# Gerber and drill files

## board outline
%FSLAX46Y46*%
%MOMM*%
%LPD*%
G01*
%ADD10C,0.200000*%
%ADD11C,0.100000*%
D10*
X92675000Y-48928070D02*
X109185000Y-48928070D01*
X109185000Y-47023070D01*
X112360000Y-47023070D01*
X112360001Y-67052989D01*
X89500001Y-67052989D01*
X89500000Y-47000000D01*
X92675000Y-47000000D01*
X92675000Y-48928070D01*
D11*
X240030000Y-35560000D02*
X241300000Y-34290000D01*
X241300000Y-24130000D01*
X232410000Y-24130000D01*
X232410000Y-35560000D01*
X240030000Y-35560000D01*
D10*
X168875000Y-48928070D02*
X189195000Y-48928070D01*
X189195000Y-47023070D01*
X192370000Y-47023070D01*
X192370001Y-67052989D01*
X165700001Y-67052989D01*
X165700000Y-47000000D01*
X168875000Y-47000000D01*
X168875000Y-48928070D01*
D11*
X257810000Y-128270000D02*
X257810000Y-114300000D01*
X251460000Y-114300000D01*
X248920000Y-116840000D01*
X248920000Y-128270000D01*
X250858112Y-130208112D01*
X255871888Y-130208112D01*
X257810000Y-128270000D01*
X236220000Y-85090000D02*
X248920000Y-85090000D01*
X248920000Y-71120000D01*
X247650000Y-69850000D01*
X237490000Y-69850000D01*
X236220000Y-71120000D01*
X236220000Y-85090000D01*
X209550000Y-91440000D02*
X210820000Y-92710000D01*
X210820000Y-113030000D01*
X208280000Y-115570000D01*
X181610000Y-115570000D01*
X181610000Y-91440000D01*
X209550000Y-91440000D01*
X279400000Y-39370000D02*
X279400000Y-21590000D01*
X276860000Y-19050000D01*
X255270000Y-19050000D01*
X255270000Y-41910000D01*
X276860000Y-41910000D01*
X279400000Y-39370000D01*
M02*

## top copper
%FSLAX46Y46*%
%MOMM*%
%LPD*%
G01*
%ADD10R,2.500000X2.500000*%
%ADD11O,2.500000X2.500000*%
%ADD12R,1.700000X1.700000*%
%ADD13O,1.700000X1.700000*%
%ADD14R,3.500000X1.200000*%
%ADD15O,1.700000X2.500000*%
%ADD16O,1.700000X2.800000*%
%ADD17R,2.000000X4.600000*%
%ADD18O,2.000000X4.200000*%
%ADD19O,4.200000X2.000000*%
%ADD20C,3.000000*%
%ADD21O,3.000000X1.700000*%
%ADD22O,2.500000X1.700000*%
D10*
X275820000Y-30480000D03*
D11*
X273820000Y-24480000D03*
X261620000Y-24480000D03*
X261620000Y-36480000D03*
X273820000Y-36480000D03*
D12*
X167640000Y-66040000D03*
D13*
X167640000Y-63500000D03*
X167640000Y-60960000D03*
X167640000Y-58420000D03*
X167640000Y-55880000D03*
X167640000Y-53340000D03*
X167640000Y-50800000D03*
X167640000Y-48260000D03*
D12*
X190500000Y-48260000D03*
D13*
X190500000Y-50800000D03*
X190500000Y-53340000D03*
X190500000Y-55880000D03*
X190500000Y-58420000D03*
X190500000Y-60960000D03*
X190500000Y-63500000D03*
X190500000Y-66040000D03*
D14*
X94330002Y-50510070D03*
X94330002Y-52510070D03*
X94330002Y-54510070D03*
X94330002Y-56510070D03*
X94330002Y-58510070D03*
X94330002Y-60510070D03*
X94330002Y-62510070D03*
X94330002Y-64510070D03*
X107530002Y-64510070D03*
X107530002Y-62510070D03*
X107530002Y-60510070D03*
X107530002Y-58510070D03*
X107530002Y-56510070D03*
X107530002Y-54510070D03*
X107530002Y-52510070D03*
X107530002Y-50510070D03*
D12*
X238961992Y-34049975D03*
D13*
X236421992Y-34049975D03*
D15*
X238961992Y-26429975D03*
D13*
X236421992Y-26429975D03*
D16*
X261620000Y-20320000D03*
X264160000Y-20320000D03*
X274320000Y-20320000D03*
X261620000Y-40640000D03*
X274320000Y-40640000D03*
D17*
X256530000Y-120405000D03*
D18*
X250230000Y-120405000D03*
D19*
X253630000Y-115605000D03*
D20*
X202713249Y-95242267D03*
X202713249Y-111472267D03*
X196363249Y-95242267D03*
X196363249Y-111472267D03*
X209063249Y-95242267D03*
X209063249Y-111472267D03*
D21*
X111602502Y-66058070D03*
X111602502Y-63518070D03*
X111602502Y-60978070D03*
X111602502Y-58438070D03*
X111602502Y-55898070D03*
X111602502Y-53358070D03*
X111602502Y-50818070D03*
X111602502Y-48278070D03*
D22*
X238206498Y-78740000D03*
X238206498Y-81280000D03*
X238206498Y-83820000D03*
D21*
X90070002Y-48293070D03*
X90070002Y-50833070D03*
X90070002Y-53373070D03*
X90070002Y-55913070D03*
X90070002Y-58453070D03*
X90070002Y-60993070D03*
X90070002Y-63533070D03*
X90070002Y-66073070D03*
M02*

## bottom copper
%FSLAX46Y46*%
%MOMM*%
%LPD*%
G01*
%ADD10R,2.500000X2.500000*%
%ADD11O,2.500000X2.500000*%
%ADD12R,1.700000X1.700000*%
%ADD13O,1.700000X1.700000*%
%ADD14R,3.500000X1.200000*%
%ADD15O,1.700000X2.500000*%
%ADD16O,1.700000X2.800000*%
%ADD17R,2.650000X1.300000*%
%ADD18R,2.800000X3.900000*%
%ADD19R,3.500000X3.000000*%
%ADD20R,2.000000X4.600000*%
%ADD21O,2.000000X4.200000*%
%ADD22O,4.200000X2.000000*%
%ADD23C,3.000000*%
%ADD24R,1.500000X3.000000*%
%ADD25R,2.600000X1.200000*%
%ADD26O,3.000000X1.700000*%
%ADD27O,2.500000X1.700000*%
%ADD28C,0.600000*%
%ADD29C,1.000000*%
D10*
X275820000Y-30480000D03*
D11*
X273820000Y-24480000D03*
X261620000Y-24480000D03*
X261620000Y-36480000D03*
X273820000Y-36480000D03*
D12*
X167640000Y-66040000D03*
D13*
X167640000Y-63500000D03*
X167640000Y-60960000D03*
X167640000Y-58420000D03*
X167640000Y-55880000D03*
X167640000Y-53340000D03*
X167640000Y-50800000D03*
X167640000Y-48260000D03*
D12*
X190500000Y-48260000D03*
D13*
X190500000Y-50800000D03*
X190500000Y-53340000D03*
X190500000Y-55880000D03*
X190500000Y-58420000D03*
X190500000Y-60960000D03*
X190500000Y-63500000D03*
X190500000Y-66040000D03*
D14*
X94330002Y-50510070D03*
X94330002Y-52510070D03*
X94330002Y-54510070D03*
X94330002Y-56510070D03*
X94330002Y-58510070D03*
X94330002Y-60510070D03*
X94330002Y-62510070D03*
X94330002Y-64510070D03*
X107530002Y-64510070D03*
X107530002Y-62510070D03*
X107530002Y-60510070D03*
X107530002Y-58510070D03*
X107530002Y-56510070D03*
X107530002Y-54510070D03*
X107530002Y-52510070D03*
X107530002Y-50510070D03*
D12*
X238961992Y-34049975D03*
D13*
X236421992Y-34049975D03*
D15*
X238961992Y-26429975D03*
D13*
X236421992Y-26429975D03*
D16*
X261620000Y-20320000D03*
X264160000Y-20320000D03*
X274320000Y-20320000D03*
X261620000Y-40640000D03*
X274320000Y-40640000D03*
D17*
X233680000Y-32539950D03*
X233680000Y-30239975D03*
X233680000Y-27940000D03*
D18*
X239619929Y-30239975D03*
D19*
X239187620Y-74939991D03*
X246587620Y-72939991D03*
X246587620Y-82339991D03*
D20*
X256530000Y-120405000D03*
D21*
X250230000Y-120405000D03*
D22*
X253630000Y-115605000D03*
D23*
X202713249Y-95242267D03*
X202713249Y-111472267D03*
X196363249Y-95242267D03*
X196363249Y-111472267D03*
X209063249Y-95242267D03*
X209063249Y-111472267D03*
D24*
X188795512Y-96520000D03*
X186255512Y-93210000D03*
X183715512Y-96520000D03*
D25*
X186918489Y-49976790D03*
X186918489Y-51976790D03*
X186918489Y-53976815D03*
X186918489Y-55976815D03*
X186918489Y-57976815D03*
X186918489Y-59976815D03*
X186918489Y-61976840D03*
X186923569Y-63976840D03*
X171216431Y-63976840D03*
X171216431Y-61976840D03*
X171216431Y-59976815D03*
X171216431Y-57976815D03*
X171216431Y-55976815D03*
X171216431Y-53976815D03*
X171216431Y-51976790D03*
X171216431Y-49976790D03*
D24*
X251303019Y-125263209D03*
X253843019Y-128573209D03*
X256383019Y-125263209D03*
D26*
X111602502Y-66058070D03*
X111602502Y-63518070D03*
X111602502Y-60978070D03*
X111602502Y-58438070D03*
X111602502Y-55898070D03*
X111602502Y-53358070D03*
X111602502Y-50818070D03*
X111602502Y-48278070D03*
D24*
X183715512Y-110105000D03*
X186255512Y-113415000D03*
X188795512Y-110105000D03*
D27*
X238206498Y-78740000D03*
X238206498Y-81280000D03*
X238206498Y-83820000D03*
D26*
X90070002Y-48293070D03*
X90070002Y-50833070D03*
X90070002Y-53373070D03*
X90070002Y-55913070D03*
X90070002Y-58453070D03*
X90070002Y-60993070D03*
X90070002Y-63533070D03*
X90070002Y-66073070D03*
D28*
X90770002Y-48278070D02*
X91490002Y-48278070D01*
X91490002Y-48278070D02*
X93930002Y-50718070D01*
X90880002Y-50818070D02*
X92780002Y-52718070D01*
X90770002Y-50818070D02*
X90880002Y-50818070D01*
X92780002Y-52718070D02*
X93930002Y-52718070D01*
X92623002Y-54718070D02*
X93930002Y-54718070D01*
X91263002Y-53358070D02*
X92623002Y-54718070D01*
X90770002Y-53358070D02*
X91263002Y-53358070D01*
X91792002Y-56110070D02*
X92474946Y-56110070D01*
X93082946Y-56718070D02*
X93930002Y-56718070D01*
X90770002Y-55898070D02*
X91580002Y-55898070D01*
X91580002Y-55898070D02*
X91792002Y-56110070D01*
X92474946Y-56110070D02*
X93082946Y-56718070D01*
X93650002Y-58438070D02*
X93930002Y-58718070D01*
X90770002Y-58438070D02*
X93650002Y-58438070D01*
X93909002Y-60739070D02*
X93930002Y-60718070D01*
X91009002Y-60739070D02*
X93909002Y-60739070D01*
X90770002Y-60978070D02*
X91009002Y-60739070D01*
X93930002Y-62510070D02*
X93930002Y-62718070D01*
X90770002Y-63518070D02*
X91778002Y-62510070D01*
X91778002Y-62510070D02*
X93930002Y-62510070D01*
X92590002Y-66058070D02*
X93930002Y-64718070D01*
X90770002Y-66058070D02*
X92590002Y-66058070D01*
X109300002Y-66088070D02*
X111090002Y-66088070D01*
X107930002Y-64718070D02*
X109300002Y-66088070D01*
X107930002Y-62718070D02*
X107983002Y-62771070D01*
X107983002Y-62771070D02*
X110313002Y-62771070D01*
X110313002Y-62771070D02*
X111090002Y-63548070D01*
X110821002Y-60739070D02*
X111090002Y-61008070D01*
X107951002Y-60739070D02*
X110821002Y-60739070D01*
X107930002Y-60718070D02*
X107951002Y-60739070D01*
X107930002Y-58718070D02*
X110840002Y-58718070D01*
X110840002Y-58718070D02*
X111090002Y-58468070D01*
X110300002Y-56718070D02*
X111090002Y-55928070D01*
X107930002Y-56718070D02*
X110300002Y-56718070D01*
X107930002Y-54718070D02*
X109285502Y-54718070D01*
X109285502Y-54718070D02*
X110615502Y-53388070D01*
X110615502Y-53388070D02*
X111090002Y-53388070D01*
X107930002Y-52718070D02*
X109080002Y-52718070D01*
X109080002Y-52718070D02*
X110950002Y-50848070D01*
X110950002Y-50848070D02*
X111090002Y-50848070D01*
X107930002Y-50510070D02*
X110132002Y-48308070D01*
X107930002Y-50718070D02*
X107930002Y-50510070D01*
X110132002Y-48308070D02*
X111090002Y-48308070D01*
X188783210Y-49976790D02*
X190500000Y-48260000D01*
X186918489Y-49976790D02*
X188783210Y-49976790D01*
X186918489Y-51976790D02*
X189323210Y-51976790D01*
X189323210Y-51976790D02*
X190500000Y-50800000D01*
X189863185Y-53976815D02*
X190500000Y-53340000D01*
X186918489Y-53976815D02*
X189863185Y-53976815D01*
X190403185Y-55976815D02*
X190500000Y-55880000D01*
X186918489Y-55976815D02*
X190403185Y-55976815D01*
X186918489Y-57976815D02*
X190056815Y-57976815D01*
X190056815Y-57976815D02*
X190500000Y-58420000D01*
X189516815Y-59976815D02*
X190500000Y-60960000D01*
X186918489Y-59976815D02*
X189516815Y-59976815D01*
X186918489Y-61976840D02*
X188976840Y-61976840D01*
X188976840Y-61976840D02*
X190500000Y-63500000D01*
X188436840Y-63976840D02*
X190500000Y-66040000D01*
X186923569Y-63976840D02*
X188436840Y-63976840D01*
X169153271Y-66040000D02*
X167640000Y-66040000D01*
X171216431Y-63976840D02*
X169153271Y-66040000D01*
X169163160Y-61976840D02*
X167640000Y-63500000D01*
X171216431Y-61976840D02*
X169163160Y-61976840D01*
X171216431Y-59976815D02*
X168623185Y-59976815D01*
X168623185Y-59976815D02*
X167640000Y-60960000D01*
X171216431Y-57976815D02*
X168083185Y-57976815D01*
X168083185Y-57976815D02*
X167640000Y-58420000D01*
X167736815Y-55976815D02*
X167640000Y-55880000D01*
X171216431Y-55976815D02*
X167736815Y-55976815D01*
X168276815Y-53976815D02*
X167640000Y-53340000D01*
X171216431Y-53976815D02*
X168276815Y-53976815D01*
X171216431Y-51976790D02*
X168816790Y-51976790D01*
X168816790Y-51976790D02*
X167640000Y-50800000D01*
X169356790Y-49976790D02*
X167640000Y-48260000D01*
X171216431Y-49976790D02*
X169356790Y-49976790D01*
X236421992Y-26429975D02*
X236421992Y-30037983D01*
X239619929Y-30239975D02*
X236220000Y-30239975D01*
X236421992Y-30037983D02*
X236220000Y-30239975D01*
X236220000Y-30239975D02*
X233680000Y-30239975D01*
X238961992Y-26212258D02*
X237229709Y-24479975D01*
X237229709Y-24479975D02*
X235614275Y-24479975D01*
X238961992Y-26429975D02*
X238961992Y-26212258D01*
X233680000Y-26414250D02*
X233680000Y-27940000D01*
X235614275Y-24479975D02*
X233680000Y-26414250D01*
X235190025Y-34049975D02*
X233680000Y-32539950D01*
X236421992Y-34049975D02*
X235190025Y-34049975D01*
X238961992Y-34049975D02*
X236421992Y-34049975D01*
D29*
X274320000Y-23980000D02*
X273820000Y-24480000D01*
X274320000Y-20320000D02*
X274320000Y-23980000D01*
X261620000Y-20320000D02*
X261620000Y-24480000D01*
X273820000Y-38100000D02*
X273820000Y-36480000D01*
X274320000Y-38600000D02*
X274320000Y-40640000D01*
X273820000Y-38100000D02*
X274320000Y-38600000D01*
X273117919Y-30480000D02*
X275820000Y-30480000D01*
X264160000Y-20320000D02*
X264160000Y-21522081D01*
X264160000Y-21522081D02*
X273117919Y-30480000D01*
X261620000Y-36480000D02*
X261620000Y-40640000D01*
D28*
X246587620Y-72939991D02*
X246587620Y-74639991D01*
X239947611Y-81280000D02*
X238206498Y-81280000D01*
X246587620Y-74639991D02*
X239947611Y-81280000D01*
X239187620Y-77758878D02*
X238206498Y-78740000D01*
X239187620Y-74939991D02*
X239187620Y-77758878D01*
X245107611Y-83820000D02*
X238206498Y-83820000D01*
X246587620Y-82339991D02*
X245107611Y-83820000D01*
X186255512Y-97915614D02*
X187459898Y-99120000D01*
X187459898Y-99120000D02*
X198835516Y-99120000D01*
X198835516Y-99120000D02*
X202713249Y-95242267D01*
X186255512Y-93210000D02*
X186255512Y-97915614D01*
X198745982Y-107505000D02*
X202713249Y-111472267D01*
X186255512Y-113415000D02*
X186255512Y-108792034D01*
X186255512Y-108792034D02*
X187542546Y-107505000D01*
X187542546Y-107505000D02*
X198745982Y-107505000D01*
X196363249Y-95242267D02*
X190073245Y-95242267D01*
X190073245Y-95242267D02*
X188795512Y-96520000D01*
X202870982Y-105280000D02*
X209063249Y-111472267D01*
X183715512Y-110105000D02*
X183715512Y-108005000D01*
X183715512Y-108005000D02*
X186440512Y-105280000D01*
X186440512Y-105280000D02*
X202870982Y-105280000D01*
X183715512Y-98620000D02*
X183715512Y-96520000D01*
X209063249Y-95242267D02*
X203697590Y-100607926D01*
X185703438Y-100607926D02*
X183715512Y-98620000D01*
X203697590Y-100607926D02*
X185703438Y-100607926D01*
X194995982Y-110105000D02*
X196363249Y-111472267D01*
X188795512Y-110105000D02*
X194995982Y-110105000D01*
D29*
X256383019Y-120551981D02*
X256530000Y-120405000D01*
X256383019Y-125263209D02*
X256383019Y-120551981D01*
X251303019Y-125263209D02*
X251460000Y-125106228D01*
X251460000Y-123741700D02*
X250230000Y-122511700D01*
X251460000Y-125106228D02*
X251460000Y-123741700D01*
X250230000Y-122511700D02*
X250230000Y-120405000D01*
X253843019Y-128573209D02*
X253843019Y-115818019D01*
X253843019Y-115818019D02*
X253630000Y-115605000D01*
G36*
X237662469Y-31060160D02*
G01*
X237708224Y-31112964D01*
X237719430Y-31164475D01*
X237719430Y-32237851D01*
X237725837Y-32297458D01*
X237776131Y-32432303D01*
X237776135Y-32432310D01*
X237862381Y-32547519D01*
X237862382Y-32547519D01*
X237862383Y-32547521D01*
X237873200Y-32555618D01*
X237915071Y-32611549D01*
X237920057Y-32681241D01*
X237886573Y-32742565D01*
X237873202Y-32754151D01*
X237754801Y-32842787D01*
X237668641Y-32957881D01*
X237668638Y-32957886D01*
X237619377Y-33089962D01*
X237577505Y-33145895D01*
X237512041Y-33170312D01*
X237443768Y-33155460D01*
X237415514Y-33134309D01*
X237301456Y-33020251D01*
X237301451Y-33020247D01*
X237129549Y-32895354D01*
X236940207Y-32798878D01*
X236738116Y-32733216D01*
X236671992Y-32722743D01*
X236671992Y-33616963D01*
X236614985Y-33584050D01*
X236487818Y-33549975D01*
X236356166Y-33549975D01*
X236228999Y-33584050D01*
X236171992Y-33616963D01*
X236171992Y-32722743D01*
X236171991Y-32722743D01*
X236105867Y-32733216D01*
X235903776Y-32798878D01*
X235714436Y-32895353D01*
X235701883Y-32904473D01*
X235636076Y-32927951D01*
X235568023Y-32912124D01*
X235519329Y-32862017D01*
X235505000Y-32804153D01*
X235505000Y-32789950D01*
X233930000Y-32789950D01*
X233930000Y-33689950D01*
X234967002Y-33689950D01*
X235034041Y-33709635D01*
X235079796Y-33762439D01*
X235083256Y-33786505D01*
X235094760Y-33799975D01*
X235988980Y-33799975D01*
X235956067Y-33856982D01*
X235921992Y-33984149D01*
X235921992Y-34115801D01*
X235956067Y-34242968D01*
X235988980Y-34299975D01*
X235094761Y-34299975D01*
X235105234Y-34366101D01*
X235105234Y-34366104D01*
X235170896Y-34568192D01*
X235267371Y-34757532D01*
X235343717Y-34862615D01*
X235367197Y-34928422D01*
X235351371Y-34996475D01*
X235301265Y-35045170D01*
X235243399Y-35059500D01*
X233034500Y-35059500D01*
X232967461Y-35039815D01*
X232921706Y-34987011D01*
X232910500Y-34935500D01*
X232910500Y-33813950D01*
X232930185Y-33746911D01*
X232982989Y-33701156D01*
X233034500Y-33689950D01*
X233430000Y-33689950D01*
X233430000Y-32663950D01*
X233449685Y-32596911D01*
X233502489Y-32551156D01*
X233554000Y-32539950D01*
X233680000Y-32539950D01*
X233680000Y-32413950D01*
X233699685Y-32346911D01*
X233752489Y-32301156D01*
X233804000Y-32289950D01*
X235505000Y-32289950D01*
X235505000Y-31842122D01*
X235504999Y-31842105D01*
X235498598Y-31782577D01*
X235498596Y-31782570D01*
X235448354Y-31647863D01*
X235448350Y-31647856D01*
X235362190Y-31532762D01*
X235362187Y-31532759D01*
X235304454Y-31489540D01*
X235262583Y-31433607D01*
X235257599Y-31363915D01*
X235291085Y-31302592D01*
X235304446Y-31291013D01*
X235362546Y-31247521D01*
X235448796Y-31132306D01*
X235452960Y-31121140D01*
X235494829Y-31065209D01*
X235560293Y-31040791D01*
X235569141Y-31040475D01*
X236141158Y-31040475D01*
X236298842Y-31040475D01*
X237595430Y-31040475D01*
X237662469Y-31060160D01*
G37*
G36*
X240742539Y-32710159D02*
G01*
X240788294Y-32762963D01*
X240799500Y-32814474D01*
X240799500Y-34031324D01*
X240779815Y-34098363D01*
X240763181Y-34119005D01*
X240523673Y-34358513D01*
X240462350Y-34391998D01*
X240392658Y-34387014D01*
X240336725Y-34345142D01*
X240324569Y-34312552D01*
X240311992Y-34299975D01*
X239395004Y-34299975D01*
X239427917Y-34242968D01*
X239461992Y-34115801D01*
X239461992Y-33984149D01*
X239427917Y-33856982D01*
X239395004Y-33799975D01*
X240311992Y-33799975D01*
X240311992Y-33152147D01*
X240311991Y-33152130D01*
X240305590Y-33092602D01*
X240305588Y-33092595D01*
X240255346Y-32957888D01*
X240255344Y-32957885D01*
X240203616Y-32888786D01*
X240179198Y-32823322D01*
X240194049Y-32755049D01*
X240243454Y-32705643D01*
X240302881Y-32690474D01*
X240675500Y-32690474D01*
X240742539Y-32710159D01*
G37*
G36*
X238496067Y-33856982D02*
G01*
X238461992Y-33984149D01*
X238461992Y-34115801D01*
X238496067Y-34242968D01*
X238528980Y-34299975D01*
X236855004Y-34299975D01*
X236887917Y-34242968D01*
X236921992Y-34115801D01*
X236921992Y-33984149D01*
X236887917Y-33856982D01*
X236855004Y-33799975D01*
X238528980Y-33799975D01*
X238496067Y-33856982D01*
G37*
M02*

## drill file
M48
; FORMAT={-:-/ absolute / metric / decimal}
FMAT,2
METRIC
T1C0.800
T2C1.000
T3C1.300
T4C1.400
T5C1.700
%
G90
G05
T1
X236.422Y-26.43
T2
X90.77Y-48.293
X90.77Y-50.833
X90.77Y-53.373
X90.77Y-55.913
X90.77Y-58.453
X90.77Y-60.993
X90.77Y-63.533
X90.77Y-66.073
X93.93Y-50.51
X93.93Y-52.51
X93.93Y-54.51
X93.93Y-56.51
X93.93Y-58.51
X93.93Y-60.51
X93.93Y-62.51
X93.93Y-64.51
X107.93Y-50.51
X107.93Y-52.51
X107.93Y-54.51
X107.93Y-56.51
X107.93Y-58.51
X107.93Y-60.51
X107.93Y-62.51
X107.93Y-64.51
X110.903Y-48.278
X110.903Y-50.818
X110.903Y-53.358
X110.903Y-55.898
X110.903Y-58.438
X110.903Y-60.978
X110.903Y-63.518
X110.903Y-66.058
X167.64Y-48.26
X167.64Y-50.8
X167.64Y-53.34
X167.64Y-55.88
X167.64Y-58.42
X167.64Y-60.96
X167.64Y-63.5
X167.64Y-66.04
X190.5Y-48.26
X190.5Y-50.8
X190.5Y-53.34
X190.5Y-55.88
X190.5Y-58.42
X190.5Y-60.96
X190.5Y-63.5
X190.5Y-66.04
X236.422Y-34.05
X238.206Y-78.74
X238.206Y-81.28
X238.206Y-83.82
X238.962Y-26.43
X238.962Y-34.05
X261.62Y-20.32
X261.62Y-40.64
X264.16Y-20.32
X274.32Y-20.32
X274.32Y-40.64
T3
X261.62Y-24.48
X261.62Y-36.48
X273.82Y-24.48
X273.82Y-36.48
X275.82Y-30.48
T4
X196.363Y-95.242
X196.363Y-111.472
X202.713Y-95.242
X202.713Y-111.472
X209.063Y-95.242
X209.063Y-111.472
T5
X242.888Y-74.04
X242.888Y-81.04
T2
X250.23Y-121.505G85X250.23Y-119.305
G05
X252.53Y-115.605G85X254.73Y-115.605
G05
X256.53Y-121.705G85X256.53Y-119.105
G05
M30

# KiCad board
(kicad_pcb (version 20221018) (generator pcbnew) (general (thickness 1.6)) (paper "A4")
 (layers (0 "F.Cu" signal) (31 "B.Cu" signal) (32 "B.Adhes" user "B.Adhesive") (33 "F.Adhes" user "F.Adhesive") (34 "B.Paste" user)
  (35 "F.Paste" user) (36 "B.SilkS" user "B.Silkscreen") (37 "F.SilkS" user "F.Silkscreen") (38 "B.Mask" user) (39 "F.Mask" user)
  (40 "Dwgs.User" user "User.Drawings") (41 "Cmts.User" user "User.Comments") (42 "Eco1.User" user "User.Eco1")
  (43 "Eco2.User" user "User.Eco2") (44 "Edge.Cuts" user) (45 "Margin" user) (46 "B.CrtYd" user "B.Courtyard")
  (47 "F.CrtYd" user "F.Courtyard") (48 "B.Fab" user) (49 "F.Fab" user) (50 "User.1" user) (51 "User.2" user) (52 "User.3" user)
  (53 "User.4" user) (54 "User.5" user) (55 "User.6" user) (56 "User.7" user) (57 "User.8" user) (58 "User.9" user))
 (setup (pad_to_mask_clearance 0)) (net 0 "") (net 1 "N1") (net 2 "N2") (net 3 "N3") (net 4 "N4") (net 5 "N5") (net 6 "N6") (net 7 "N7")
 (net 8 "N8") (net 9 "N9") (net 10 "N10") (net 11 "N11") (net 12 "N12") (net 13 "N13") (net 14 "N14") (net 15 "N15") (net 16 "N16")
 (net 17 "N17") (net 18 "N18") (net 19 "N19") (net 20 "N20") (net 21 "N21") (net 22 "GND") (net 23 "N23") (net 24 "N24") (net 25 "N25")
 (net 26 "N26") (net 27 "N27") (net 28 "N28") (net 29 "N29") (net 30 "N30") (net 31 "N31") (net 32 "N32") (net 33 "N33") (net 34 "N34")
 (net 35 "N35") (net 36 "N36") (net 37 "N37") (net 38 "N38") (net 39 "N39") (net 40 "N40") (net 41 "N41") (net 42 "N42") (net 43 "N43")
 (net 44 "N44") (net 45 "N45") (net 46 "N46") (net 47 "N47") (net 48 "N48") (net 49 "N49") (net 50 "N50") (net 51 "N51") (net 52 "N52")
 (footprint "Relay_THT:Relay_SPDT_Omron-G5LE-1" (layer "F.Cu") (at 275.82 30.48 -90)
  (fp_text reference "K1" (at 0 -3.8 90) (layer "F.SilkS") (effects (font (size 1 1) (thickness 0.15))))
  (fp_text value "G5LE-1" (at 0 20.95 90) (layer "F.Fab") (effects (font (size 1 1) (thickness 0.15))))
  (pad "1" thru_hole rect (at 0 0 270) (size 2.5 2.5) (drill 1.3) (layers "*.Cu" "*.Mask") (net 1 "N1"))
  (pad "2" thru_hole oval (at -6 2 270) (size 2.5 2.5) (drill 1.3) (layers "*.Cu" "*.Mask") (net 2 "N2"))
  (pad "3" thru_hole oval (at -6 14.2 270) (size 2.5 2.5) (drill 1.3) (layers "*.Cu" "*.Mask") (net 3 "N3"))
  (pad "4" thru_hole oval (at 6 14.2 270) (size 2.5 2.5) (drill 1.3) (layers "*.Cu" "*.Mask") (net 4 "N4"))
  (pad "5" thru_hole oval (at 6 2 270) (size 2.5 2.5) (drill 1.3) (layers "*.Cu" "*.Mask") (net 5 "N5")))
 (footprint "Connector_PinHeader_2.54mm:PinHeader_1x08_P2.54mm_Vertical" (layer "F.Cu") (at 167.64 66.04 180)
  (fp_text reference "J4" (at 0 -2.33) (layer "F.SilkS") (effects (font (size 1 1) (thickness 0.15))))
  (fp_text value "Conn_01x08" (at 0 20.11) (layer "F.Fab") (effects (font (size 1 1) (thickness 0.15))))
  (pad "1" thru_hole rect (at 0 0 180) (size 1.7 1.7) (drill 1) (layers "*.Cu" "*.Mask") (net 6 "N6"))
  (pad "2" thru_hole oval (at 0 2.54 180) (size 1.7 1.7) (drill 1) (layers "*.Cu" "*.Mask") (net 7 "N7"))
  (pad "3" thru_hole oval (at 0 5.08 180) (size 1.7 1.7) (drill 1) (layers "*.Cu" "*.Mask") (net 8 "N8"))
  (pad "4" thru_hole oval (at 0 7.62 180) (size 1.7 1.7) (drill 1) (layers "*.Cu" "*.Mask") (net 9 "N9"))
  (pad "5" thru_hole oval (at 0 10.16 180) (size 1.7 1.7) (drill 1) (layers "*.Cu" "*.Mask") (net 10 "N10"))
  (pad "6" thru_hole oval (at 0 12.7 180) (size 1.7 1.7) (drill 1) (layers "*.Cu" "*.Mask") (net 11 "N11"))
  (pad "7" thru_hole oval (at 0 15.24 180) (size 1.7 1.7) (drill 1) (layers "*.Cu" "*.Mask") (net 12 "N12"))
  (pad "8" thru_hole oval (at 0 17.78 180) (size 1.7 1.7) (drill 1) (layers "*.Cu" "*.Mask") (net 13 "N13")))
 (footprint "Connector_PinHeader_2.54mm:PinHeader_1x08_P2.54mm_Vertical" (layer "F.Cu") (at 190.5 48.26)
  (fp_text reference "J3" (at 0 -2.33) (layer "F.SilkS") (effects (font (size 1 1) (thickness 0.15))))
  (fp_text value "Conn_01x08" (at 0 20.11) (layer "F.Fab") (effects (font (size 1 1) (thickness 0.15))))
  (pad "1" thru_hole rect (at 0 0) (size 1.7 1.7) (drill 1) (layers "*.Cu" "*.Mask") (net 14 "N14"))
  (pad "2" thru_hole oval (at 0 2.54) (size 1.7 1.7) (drill 1) (layers "*.Cu" "*.Mask") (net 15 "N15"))
  (pad "3" thru_hole oval (at 0 5.08) (size 1.7 1.7) (drill 1) (layers "*.Cu" "*.Mask") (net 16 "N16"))
  (pad "4" thru_hole oval (at 0 7.62) (size 1.7 1.7) (drill 1) (layers "*.Cu" "*.Mask") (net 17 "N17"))
  (pad "5" thru_hole oval (at 0 10.16) (size 1.7 1.7) (drill 1) (layers "*.Cu" "*.Mask") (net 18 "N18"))
  (pad "6" thru_hole oval (at 0 12.7) (size 1.7 1.7) (drill 1) (layers "*.Cu" "*.Mask") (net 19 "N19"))
  (pad "7" thru_hole oval (at 0 15.24) (size 1.7 1.7) (drill 1) (layers "*.Cu" "*.Mask") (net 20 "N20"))
  (pad "8" thru_hole oval (at 0 17.78) (size 1.7 1.7) (drill 1) (layers "*.Cu" "*.Mask") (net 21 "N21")))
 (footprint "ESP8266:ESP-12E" (layer "F.Cu") (at 93.930002 50.51007)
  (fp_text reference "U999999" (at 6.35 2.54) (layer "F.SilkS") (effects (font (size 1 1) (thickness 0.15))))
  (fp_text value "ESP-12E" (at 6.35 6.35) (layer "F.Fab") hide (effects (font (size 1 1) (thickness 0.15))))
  (pad "1" thru_hole rect (at 0 0) (size 3.5 1.2) (drill 1 (offset 0.4 0)) (layers "*.Cu" "*.Mask" "F.SilkS"))
  (pad "2" thru_hole rect (at 0 2) (size 3.5 1.2) (drill 1 (offset 0.4 0)) (layers "*.Cu" "*.Mask" "F.SilkS"))
  (pad "3" thru_hole rect (at 0 4) (size 3.5 1.2) (drill 1 (offset 0.4 0)) (layers "*.Cu" "*.Mask" "F.SilkS"))
  (pad "4" thru_hole rect (at 0 6) (size 3.5 1.2) (drill 1 (offset 0.4 0)) (layers "*.Cu" "*.Mask" "F.SilkS"))
  (pad "5" thru_hole rect (at 0 8) (size 3.5 1.2) (drill 1 (offset 0.4 0)) (layers "*.Cu" "*.Mask" "F.SilkS"))
  (pad "6" thru_hole rect (at 0 10) (size 3.5 1.2) (drill 1 (offset 0.4 0)) (layers "*.Cu" "*.Mask" "F.SilkS"))
  (pad "7" thru_hole rect (at 0 12) (size 3.5 1.2) (drill 1 (offset 0.4 0)) (layers "*.Cu" "*.Mask" "F.SilkS"))
  (pad "8" thru_hole rect (at 0 14) (size 3.5 1.2) (drill 1 (offset 0.4 0)) (layers "*.Cu" "*.Mask" "F.SilkS"))
  (pad "9" thru_hole rect (at 14 14 180) (size 3.5 1.2) (drill 1 (offset 0.4 0)) (layers "*.Cu" "*.Mask" "F.SilkS"))
  (pad "10" thru_hole rect (at 14 12 180) (size 3.5 1.2) (drill 1 (offset 0.4 0)) (layers "*.Cu" "*.Mask" "F.SilkS"))
  (pad "11" thru_hole rect (at 14 10 180) (size 3.5 1.2) (drill 1 (offset 0.4 0)) (layers "*.Cu" "*.Mask" "F.SilkS"))
  (pad "12" thru_hole rect (at 14 8 180) (size 3.5 1.2) (drill 1 (offset 0.4 0)) (layers "*.Cu" "*.Mask" "F.SilkS"))
  (pad "13" thru_hole rect (at 14 6 180) (size 3.5 1.2) (drill 1 (offset 0.4 0)) (layers "*.Cu" "*.Mask" "F.SilkS"))
  (pad "14" thru_hole rect (at 14 4 180) (size 3.5 1.2) (drill 1 (offset 0.4 0)) (layers "*.Cu" "*.Mask" "F.SilkS"))
  (pad "15" thru_hole rect (at 14 2 180) (size 3.5 1.2) (drill 1 (offset 0.4 0)) (layers "*.Cu" "*.Mask" "F.SilkS"))
  (pad "16" thru_hole rect (at 14 0 180) (size 3.5 1.2) (drill 1 (offset 0.4 0)) (layers "*.Cu" "*.Mask" "F.SilkS")))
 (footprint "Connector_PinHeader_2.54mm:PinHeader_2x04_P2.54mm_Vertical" (layer "F.Cu") (at 238.961992 34.049975 180)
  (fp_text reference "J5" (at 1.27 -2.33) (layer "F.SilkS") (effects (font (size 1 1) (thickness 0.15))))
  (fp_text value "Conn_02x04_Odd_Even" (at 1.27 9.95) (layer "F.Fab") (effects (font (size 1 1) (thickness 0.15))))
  (pad "1" thru_hole rect (at 0 0 180) (size 1.7 1.7) (drill 1) (layers "*.Cu" "*.Mask") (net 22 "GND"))
  (pad "2" thru_hole oval (at 2.54 0 180) (size 1.7 1.7) (drill 1) (layers "*.Cu" "*.Mask") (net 22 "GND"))
  (pad "7" thru_hole oval (at 0 7.62 180) (size 1.7 2.5) (drill 1) (layers "*.Cu" "*.Mask") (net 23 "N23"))
  (pad "8" thru_hole oval (at 2.54 7.62 180) (size 1.7 1.7) (drill 0.8) (layers "*.Cu" "*.Mask") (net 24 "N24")))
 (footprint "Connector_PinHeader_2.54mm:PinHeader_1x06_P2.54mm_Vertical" (layer "F.Cu") (at 261.62 20.32 90)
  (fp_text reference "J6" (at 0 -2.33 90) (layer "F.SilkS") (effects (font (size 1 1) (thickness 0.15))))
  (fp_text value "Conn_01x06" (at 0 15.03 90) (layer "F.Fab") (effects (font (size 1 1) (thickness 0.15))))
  (pad "1" thru_hole oval (at 0 0 90) (size 2.8 1.7) (drill 1) (layers "*.Cu" "*.Mask") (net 3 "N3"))
  (pad "2" thru_hole oval (at 0 2.54 90) (size 2.8 1.7) (drill 1) (layers "*.Cu" "*.Mask") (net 1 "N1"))
  (pad "6" thru_hole oval (at 0 12.7 90) (size 2.8 1.7) (drill 1) (layers "*.Cu" "*.Mask") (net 2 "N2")))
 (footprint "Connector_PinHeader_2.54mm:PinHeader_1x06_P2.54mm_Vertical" (layer "F.Cu") (at 261.62 40.64 90)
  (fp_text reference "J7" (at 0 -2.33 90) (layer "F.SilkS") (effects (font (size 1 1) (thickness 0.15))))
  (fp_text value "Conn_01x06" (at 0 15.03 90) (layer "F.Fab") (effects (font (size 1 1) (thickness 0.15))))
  (pad "1" thru_hole oval (at 0 0 90) (size 2.8 1.7) (drill 1) (layers "*.Cu" "*.Mask") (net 4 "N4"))
  (pad "6" thru_hole oval (at 0 12.7 90) (size 2.8 1.7) (drill 1) (layers "*.Cu" "*.Mask") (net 5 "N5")))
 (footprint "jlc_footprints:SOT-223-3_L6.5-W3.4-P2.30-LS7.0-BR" (layer "B.Cu") (at 236.649952 30.239975 180)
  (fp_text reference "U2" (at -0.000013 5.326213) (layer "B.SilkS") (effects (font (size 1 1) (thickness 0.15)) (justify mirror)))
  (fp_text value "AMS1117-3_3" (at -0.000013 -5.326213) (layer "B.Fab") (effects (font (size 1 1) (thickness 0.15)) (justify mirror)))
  (pad "1" smd rect (at 2.969952 -2.299975 180) (size 2.65 1.3) (layers "B.Cu" "B.Paste" "B.Mask") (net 22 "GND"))
  (pad "2" smd rect (at 2.969952 0 180) (size 2.65 1.3) (layers "B.Cu" "B.Paste" "B.Mask") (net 24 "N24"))
  (pad "3" smd rect (at 2.969952 2.299975 180) (size 2.65 1.3) (layers "B.Cu" "B.Paste" "B.Mask") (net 23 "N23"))
  (pad "4" smd rect (at -2.969977 0 180) (size 2.8 3.9) (layers "B.Cu" "B.Paste" "B.Mask") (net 24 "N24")))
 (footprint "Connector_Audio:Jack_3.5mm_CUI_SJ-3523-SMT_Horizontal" (layer "B.Cu") (at 242.88762 76.539991 180)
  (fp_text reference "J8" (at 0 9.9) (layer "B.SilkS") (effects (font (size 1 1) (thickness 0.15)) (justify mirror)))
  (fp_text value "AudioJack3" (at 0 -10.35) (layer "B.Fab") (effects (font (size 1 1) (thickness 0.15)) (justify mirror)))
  (pad "" np_thru_hole circle (at 0 -4.5 180) (size 1.7 1.7) (drill 1.7) (layers "*.Cu" "*.Mask"))
  (pad "" np_thru_hole circle (at 0 2.5 180) (size 1.7 1.7) (drill 1.7) (layers "*.Cu" "*.Mask"))
  (pad "R" smd rect (at 3.7 1.6 180) (size 3.5 3) (layers "B.Cu" "B.Paste" "B.Mask") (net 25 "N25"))
  (pad "S" smd rect (at -3.7 3.6 180) (size 3.5 3) (layers "B.Cu" "B.Paste" "B.Mask") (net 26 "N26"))
  (pad "T" smd rect (at -3.7 -5.8 180) (size 3.5 3) (layers "B.Cu" "B.Paste" "B.Mask") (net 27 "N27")))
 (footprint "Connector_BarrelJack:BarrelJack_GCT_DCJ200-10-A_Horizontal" (layer "B.Cu") (at 256.53 120.405 90)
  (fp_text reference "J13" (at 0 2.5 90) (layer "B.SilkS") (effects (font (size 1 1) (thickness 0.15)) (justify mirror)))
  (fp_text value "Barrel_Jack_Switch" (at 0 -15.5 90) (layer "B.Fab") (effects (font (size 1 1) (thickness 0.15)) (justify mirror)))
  (pad "1" thru_hole rect (at 0 0 90) (size 4.6 2) (drill oval 3.6 1) (layers "*.Cu" "*.Mask") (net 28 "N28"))
  (pad "2" thru_hole oval (at 0 -6.3 90) (size 4.2 2) (drill oval 3.2 1) (layers "*.Cu" "*.Mask") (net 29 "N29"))
  (pad "3" thru_hole oval (at 4.8 -2.9 90) (size 2 4.2) (drill oval 1 3.2) (layers "*.Cu" "*.Mask") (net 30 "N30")))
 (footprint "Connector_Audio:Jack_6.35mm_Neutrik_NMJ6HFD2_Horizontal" (layer "B.Cu") (at 209.063249 95.242267 180)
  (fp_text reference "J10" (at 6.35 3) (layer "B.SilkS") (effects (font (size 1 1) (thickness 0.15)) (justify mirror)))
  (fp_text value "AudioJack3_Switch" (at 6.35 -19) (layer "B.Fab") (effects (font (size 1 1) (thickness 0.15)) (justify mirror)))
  (pad "R" thru_hole circle (at 6.35 0 180) (size 3 3) (drill 1.4) (layers "*.Cu" "*.Mask") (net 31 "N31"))
  (pad "RN" thru_hole circle (at 6.35 -16.23 180) (size 3 3) (drill 1.4) (layers "*.Cu" "*.Mask") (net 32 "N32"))
  (pad "S" thru_hole circle (at 12.7 0 180) (size 3 3) (drill 1.4) (layers "*.Cu" "*.Mask") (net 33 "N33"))
  (pad "SN" thru_hole circle (at 12.7 -16.23 180) (size 3 3) (drill 1.4) (layers "*.Cu" "*.Mask") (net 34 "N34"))
  (pad "T" thru_hole circle (at 0 0 180) (size 3 3) (drill 1.4) (layers "*.Cu" "*.Mask") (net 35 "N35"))
  (pad "TN" thru_hole circle (at 0 -16.23 180) (size 3 3) (drill 1.4) (layers "*.Cu" "*.Mask") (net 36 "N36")))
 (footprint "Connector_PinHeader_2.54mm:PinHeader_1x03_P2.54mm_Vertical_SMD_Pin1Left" (layer "B.Cu") (at 186.255512 94.865 90)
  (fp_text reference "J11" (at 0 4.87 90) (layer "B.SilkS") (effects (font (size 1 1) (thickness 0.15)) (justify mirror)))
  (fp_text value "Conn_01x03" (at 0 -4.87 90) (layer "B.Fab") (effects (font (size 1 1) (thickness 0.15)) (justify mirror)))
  (pad "1" smd rect (at -1.655 2.54 90) (size 3 1.5) (layers "B.Cu" "B.Paste" "B.Mask") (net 33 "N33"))
  (pad "2" smd rect (at 1.655 0 90) (size 3 1.5) (layers "B.Cu" "B.Paste" "B.Mask") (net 31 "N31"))
  (pad "3" smd rect (at -1.655 -2.54 90) (size 3 1.5) (layers "B.Cu" "B.Paste" "B.Mask") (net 35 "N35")))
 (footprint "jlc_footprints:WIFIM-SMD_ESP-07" (layer "B.Cu") (at 179.07 56.976815 -90)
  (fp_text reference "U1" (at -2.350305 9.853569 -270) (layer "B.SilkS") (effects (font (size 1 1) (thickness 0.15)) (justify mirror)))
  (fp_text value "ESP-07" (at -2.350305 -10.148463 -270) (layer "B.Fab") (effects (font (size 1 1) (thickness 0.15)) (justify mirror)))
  (pad "1" smd rect (at -7.000025 -7.848489 270) (size 1.2 2.6) (layers "B.Cu" "B.Paste" "B.Mask") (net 14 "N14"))
  (pad "2" smd rect (at -5.000025 -7.848489 270) (size 1.2 2.6) (layers "B.Cu" "B.Paste" "B.Mask") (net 15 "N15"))
  (pad "3" smd rect (at -3 -7.848489 270) (size 1.2 2.6) (layers "B.Cu" "B.Paste" "B.Mask") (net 16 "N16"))
  (pad "4" smd rect (at -1 -7.848489 270) (size 1.2 2.6) (layers "B.Cu" "B.Paste" "B.Mask") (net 17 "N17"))
  (pad "5" smd rect (at 1 -7.848489 270) (size 1.2 2.6) (layers "B.Cu" "B.Paste" "B.Mask") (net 18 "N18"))
  (pad "6" smd rect (at 3 -7.848489 270) (size 1.2 2.6) (layers "B.Cu" "B.Paste" "B.Mask") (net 19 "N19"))
  (pad "7" smd rect (at 5.000025 -7.848489 270) (size 1.2 2.6) (layers "B.Cu" "B.Paste" "B.Mask") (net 20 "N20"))
  (pad "8" smd rect (at 7.000025 -7.853569 270) (size 1.2 2.6) (layers "B.Cu" "B.Paste" "B.Mask") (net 21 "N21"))
  (pad "9" smd rect (at 7.000025 7.853569 270) (size 1.2 2.6) (layers "B.Cu" "B.Paste" "B.Mask") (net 6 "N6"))
  (pad "10" smd rect (at 5.000025 7.853569 270) (size 1.2 2.6) (layers "B.Cu" "B.Paste" "B.Mask") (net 7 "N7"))
  (pad "11" smd rect (at 3 7.853569 270) (size 1.2 2.6) (layers "B.Cu" "B.Paste" "B.Mask") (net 8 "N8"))
  (pad "12" smd rect (at 1 7.853569 270) (size 1.2 2.6) (layers "B.Cu" "B.Paste" "B.Mask") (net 9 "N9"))
  (pad "13" smd rect (at -1 7.853569 270) (size 1.2 2.6) (layers "B.Cu" "B.Paste" "B.Mask") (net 10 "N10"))
  (pad "14" smd rect (at -3 7.853569 270) (size 1.2 2.6) (layers "B.Cu" "B.Paste" "B.Mask") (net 11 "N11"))
  (pad "15" smd rect (at -5.000025 7.853569 270) (size 1.2 2.6) (layers "B.Cu" "B.Paste" "B.Mask") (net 12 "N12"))
  (pad "16" smd rect (at -7.000025 7.853569 270) (size 1.2 2.6) (layers "B.Cu" "B.Paste" "B.Mask") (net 13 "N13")))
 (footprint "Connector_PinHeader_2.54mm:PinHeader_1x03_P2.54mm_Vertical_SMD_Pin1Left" (layer "B.Cu") (at 253.843019 126.918209 -90)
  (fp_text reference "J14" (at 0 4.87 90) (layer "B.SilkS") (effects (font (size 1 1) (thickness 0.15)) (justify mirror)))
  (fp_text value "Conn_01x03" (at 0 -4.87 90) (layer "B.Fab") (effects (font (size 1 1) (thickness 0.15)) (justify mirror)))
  (pad "1" smd rect (at -1.655 2.54 270) (size 3 1.5) (layers "B.Cu" "B.Paste" "B.Mask") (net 29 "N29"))
  (pad "2" smd rect (at 1.655 0 270) (size 3 1.5) (layers "B.Cu" "B.Paste" "B.Mask") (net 30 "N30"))
  (pad "3" smd rect (at -1.655 -2.54 270) (size 3 1.5) (layers "B.Cu" "B.Paste" "B.Mask") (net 28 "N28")))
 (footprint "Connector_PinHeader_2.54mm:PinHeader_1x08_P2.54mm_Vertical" (layer "B.Cu") (at 110.902502 66.05807)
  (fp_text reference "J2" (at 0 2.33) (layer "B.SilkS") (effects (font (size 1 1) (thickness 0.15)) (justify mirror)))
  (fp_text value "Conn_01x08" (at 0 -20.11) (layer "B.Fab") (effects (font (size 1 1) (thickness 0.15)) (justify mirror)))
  (pad "1" thru_hole oval (at 0 0) (size 3 1.7) (drill 1 (offset 0.7 0)) (layers "*.Cu" "*.Mask") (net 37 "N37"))
  (pad "2" thru_hole oval (at 0 -2.54) (size 3 1.7) (drill 1 (offset 0.7 0)) (layers "*.Cu" "*.Mask") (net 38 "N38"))
  (pad "3" thru_hole oval (at 0 -5.08) (size 3 1.7) (drill 1 (offset 0.7 0)) (layers "*.Cu" "*.Mask") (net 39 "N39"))
  (pad "4" thru_hole oval (at 0 -7.62) (size 3 1.7) (drill 1 (offset 0.7 0)) (layers "*.Cu" "*.Mask") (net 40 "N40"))
  (pad "5" thru_hole oval (at 0 -10.16) (size 3 1.7) (drill 1 (offset 0.7 0)) (layers "*.Cu" "*.Mask") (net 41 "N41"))
  (pad "6" thru_hole oval (at 0 -12.7) (size 3 1.7) (drill 1 (offset 0.7 0)) (layers "*.Cu" "*.Mask") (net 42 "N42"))
  (pad "7" thru_hole oval (at 0 -15.24) (size 3 1.7) (drill 1 (offset 0.7 0)) (layers "*.Cu" "*.Mask") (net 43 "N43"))
  (pad "8" thru_hole oval (at 0 -17.78) (size 3 1.7) (drill 1 (offset 0.7 0)) (layers "*.Cu" "*.Mask") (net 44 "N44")))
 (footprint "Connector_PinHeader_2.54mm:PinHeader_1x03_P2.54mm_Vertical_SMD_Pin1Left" (layer "B.Cu") (at 186.255512 111.76 -90)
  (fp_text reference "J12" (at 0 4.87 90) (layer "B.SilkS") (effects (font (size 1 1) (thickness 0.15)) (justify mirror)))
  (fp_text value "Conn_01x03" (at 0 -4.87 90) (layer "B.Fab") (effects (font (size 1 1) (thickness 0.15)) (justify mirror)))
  (pad "1" smd rect (at -1.655 2.54 270) (size 3 1.5) (layers "B.Cu" "B.Paste" "B.Mask") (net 36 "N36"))
  (pad "2" smd rect (at 1.655 0 270) (size 3 1.5) (layers "B.Cu" "B.Paste" "B.Mask") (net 32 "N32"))
  (pad "3" smd rect (at -1.655 -2.54 270) (size 3 1.5) (layers "B.Cu" "B.Paste" "B.Mask") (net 34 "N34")))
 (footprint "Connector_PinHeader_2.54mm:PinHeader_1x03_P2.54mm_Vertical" (layer "B.Cu") (at 238.206498 78.74 180)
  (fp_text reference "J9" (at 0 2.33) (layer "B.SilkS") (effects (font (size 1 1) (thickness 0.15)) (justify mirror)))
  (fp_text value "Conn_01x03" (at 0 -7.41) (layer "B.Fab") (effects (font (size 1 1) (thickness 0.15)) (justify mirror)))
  (pad "1" thru_hole oval (at 0 0 180) (size 2.5 1.7) (drill 1) (layers "*.Cu" "*.Mask") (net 25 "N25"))
  (pad "2" thru_hole oval (at 0 -2.54 180) (size 2.5 1.7) (drill 1) (layers "*.Cu" "*.Mask") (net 26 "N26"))
  (pad "3" thru_hole oval (at 0 -5.08 180) (size 2.5 1.7) (drill 1) (layers "*.Cu" "*.Mask") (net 27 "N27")))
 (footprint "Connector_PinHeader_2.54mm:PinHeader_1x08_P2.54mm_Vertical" (layer "B.Cu") (at 90.770002 48.29307 180)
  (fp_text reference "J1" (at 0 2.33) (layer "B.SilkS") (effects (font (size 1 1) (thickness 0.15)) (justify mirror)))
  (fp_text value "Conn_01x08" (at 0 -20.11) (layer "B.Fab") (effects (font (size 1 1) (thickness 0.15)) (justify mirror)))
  (pad "1" thru_hole oval (at 0 0 180) (size 3 1.7) (drill 1 (offset 0.7 0)) (layers "*.Cu" "*.Mask") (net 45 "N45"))
  (pad "2" thru_hole oval (at 0 -2.54 180) (size 3 1.7) (drill 1 (offset 0.7 0)) (layers "*.Cu" "*.Mask") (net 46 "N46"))
  (pad "3" thru_hole oval (at 0 -5.08 180) (size 3 1.7) (drill 1 (offset 0.7 0)) (layers "*.Cu" "*.Mask") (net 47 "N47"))
  (pad "4" thru_hole oval (at 0 -7.62 180) (size 3 1.7) (drill 1 (offset 0.7 0)) (layers "*.Cu" "*.Mask") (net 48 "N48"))
  (pad "5" thru_hole oval (at 0 -10.16 180) (size 3 1.7) (drill 1 (offset 0.7 0)) (layers "*.Cu" "*.Mask") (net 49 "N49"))
  (pad "6" thru_hole oval (at 0 -12.7 180) (size 3 1.7) (drill 1 (offset 0.7 0)) (layers "*.Cu" "*.Mask") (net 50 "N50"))
  (pad "7" thru_hole oval (at 0 -15.24 180) (size 3 1.7) (drill 1 (offset 0.7 0)) (layers "*.Cu" "*.Mask") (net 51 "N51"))
  (pad "8" thru_hole oval (at 0 -17.78 180) (size 3 1.7) (drill 1 (offset 0.7 0)) (layers "*.Cu" "*.Mask") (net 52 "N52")))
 (gr_poly
  (pts (xy 92.675 48.92807) (xy 109.185 48.92807) (xy 109.185 47.02307) (xy 112.36 47.02307) (xy 112.360001 67.052989)
   (xy 89.500001 67.052989) (xy 89.5 47) (xy 92.675 47))
  (stroke (width 0.2) (type solid)) (fill none) (layer "Edge.Cuts"))
 (gr_poly
  (pts (xy 240.03 35.56) (xy 241.3 34.29) (xy 241.3 24.13) (xy 232.41 24.13) (xy 232.41 35.56)) (stroke (width 0.1) (type solid))
  (fill none) (layer "Edge.Cuts"))
 (gr_poly
  (pts (xy 168.875 48.92807) (xy 189.195 48.92807) (xy 189.195 47.02307) (xy 192.37 47.02307) (xy 192.370001 67.052989)
   (xy 165.700001 67.052989) (xy 165.7 47) (xy 168.875 47))
  (stroke (width 0.2) (type solid)) (fill none) (layer "Edge.Cuts"))
 (gr_poly
  (pts (xy 257.81 128.27) (xy 257.81 114.3) (xy 251.46 114.3) (xy 248.92 116.84) (xy 248.92 128.27) (xy 250.858112 130.208112)
   (xy 255.871888 130.208112))
  (stroke (width 0.1) (type solid)) (fill none) (layer "Edge.Cuts"))
 (gr_poly
  (pts (xy 236.22 85.09) (xy 248.92 85.09) (xy 248.92 71.12) (xy 247.65 69.85) (xy 237.49 69.85) (xy 236.22 71.12))
  (stroke (width 0.1) (type solid)) (fill none) (layer "Edge.Cuts"))
 (gr_poly
  (pts (xy 209.55 91.44) (xy 210.82 92.71) (xy 210.82 113.03) (xy 208.28 115.57) (xy 181.61 115.57) (xy 181.61 91.44))
  (stroke (width 0.1) (type solid)) (fill none) (layer "Edge.Cuts"))
 (gr_poly
  (pts (xy 279.4 39.37) (xy 279.4 21.59) (xy 276.86 19.05) (xy 255.27 19.05) (xy 255.27 41.91) (xy 276.86 41.91))
  (stroke (width 0.1) (type solid)) (fill none) (layer "Edge.Cuts"))
 (segment (start 90.770002 48.27807) (end 91.490002 48.27807) (width 0.6) (layer "B.Cu") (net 45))
 (segment (start 91.490002 48.27807) (end 93.930002 50.71807) (width 0.6) (layer "B.Cu") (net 45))
 (segment (start 90.880002 50.81807) (end 92.780002 52.71807) (width 0.6) (layer "B.Cu") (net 46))
 (segment (start 90.770002 50.81807) (end 90.880002 50.81807) (width 0.6) (layer "B.Cu") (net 46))
 (segment (start 92.780002 52.71807) (end 93.930002 52.71807) (width 0.6) (layer "B.Cu") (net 46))
 (segment (start 92.623002 54.71807) (end 93.930002 54.71807) (width 0.6) (layer "B.Cu") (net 47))
 (segment (start 91.263002 53.35807) (end 92.623002 54.71807) (width 0.6) (layer "B.Cu") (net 47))
 (segment (start 90.770002 53.35807) (end 91.263002 53.35807) (width 0.6) (layer "B.Cu") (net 47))
 (segment (start 91.792002 56.11007) (end 92.474946 56.11007) (width 0.6) (layer "B.Cu") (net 48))
 (segment (start 93.082946 56.71807) (end 93.930002 56.71807) (width 0.6) (layer "B.Cu") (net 48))
 (segment (start 90.770002 55.89807) (end 91.580002 55.89807) (width 0.6) (layer "B.Cu") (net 48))
 (segment (start 91.580002 55.89807) (end 91.792002 56.11007) (width 0.6) (layer "B.Cu") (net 48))
 (segment (start 92.474946 56.11007) (end 93.082946 56.71807) (width 0.6) (layer "B.Cu") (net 48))
 (segment (start 93.650002 58.43807) (end 93.930002 58.71807) (width 0.6) (layer "B.Cu") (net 49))
 (segment (start 90.770002 58.43807) (end 93.650002 58.43807) (width 0.6) (layer "B.Cu") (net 49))
 (segment (start 93.909002 60.73907) (end 93.930002 60.71807) (width 0.6) (layer "B.Cu") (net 50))
 (segment (start 91.009002 60.73907) (end 93.909002 60.73907) (width 0.6) (layer "B.Cu") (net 50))
 (segment (start 90.770002 60.97807) (end 91.009002 60.73907) (width 0.6) (layer "B.Cu") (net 50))
 (segment (start 93.930002 62.51007) (end 93.930002 62.71807) (width 0.6) (layer "B.Cu") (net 51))
 (segment (start 90.770002 63.51807) (end 91.778002 62.51007) (width 0.6) (layer "B.Cu") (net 51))
 (segment (start 91.778002 62.51007) (end 93.930002 62.51007) (width 0.6) (layer "B.Cu") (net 51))
 (segment (start 92.590002 66.05807) (end 93.930002 64.71807) (width 0.6) (layer "B.Cu") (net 52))
 (segment (start 90.770002 66.05807) (end 92.590002 66.05807) (width 0.6) (layer "B.Cu") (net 52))
 (segment (start 109.300002 66.08807) (end 111.090002 66.08807) (width 0.6) (layer "B.Cu") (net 37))
 (segment (start 107.930002 64.71807) (end 109.300002 66.08807) (width 0.6) (layer "B.Cu") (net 37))
 (segment (start 107.930002 62.71807) (end 107.983002 62.77107) (width 0.6) (layer "B.Cu") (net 38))
 (segment (start 107.983002 62.77107) (end 110.313002 62.77107) (width 0.6) (layer "B.Cu") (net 38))
 (segment (start 110.313002 62.77107) (end 111.090002 63.54807) (width 0.6) (layer "B.Cu") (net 38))
 (segment (start 110.821002 60.73907) (end 111.090002 61.00807) (width 0.6) (layer "B.Cu") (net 39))
 (segment (start 107.951002 60.73907) (end 110.821002 60.73907) (width 0.6) (layer "B.Cu") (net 39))
 (segment (start 107.930002 60.71807) (end 107.951002 60.73907) (width 0.6) (layer "B.Cu") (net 39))
 (segment (start 107.930002 58.71807) (end 110.840002 58.71807) (width 0.6) (layer "B.Cu") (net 40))
 (segment (start 110.840002 58.71807) (end 111.090002 58.46807) (width 0.6) (layer "B.Cu") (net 40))
 (segment (start 110.300002 56.71807) (end 111.090002 55.92807) (width 0.6) (layer "B.Cu") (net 41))
 (segment (start 107.930002 56.71807) (end 110.300002 56.71807) (width 0.6) (layer "B.Cu") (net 41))
 (segment (start 107.930002 54.71807) (end 109.285502 54.71807) (width 0.6) (layer "B.Cu") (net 42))
 (segment (start 109.285502 54.71807) (end 110.615502 53.38807) (width 0.6) (layer "B.Cu") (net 42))
 (segment (start 110.615502 53.38807) (end 111.090002 53.38807) (width 0.6) (layer "B.Cu") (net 42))
 (segment (start 107.930002 52.71807) (end 109.080002 52.71807) (width 0.6) (layer "B.Cu") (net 43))
 (segment (start 109.080002 52.71807) (end 110.950002 50.84807) (width 0.6) (layer "B.Cu") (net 43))
 (segment (start 110.950002 50.84807) (end 111.090002 50.84807) (width 0.6) (layer "B.Cu") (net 43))
 (segment (start 107.930002 50.51007) (end 110.132002 48.30807) (width 0.6) (layer "B.Cu") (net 44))
 (segment (start 107.930002 50.71807) (end 107.930002 50.51007) (width 0.6) (layer "B.Cu") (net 44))
 (segment (start 110.132002 48.30807) (end 111.090002 48.30807) (width 0.6) (layer "B.Cu") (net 44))
 (segment (start 188.78321 49.97679) (end 190.5 48.26) (width 0.6) (layer "B.Cu") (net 14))
 (segment (start 186.918489 49.97679) (end 188.78321 49.97679) (width 0.6) (layer "B.Cu") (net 14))
 (segment (start 186.918489 51.97679) (end 189.32321 51.97679) (width 0.6) (layer "B.Cu") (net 15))
 (segment (start 189.32321 51.97679) (end 190.5 50.8) (width 0.6) (layer "B.Cu") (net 15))
 (segment (start 189.863185 53.976815) (end 190.5 53.34) (width 0.6) (layer "B.Cu") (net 16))
 (segment (start 186.918489 53.976815) (end 189.863185 53.976815) (width 0.6) (layer "B.Cu") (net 16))
 (segment (start 190.403185 55.976815) (end 190.5 55.88) (width 0.6) (layer "B.Cu") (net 17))
 (segment (start 186.918489 55.976815) (end 190.403185 55.976815) (width 0.6) (layer "B.Cu") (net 17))
 (segment (start 186.918489 57.976815) (end 190.056815 57.976815) (width 0.6) (layer "B.Cu") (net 18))
 (segment (start 190.056815 57.976815) (end 190.5 58.42) (width 0.6) (layer "B.Cu") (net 18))
 (segment (start 189.516815 59.976815) (end 190.5 60.96) (width 0.6) (layer "B.Cu") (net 19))
 (segment (start 186.918489 59.976815) (end 189.516815 59.976815) (width 0.6) (layer "B.Cu") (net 19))
 (segment (start 186.918489 61.97684) (end 188.97684 61.97684) (width 0.6) (layer "B.Cu") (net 20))
 (segment (start 188.97684 61.97684) (end 190.5 63.5) (width 0.6) (layer "B.Cu") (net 20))
 (segment (start 188.43684 63.97684) (end 190.5 66.04) (width 0.6) (layer "B.Cu") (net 21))
 (segment (start 186.923569 63.97684) (end 188.43684 63.97684) (width 0.6) (layer "B.Cu") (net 21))
 (segment (start 169.153271 66.04) (end 167.64 66.04) (width 0.6) (layer "B.Cu") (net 6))
 (segment (start 171.216431 63.97684) (end 169.153271 66.04) (width 0.6) (layer "B.Cu") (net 6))
 (segment (start 169.16316 61.97684) (end 167.64 63.5) (width 0.6) (layer "B.Cu") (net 7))
 (segment (start 171.216431 61.97684) (end 169.16316 61.97684) (width 0.6) (layer "B.Cu") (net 7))
 (segment (start 171.216431 59.976815) (end 168.623185 59.976815) (width 0.6) (layer "B.Cu") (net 8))
 (segment (start 168.623185 59.976815) (end 167.64 60.96) (width 0.6) (layer "B.Cu") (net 8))
 (segment (start 171.216431 57.976815) (end 168.083185 57.976815) (width 0.6) (layer "B.Cu") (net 9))
 (segment (start 168.083185 57.976815) (end 167.64 58.42) (width 0.6) (layer "B.Cu") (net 9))
 (segment (start 167.736815 55.976815) (end 167.64 55.88) (width 0.6) (layer "B.Cu") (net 10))
 (segment (start 171.216431 55.976815) (end 167.736815 55.976815) (width 0.6) (layer "B.Cu") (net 10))
 (segment (start 168.276815 53.976815) (end 167.64 53.34) (width 0.6) (layer "B.Cu") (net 11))
 (segment (start 171.216431 53.976815) (end 168.276815 53.976815) (width 0.6) (layer "B.Cu") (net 11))
 (segment (start 171.216431 51.97679) (end 168.81679 51.97679) (width 0.6) (layer "B.Cu") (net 12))
 (segment (start 168.81679 51.97679) (end 167.64 50.8) (width 0.6) (layer "B.Cu") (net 12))
 (segment (start 169.35679 49.97679) (end 167.64 48.26) (width 0.6) (layer "B.Cu") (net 13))
 (segment (start 171.216431 49.97679) (end 169.35679 49.97679) (width 0.6) (layer "B.Cu") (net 13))
 (segment (start 236.421992 26.429975) (end 236.421992 30.037983) (width 0.6) (layer "B.Cu") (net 24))
 (segment (start 239.619929 30.239975) (end 236.22 30.239975) (width 0.6) (layer "B.Cu") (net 24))
 (segment (start 236.421992 30.037983) (end 236.22 30.239975) (width 0.6) (layer "B.Cu") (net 24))
 (segment (start 236.22 30.239975) (end 233.68 30.239975) (width 0.6) (layer "B.Cu") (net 24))
 (segment (start 238.961992 26.212258) (end 237.229709 24.479975) (width 0.6) (layer "B.Cu") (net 23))
 (segment (start 237.229709 24.479975) (end 235.614275 24.479975) (width 0.6) (layer "B.Cu") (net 23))
 (segment (start 238.961992 26.429975) (end 238.961992 26.212258) (width 0.6) (layer "B.Cu") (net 23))
 (segment (start 233.68 26.41425) (end 233.68 27.94) (width 0.6) (layer "B.Cu") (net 23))
 (segment (start 235.614275 24.479975) (end 233.68 26.41425) (width 0.6) (layer "B.Cu") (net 23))
 (segment (start 235.190025 34.049975) (end 233.68 32.53995) (width 0.6) (layer "B.Cu") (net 22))
 (segment (start 236.421992 34.049975) (end 235.190025 34.049975) (width 0.6) (layer "B.Cu") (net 22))
 (segment (start 238.961992 34.049975) (end 236.421992 34.049975) (width 0.6) (layer "B.Cu") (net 22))
 (segment (start 274.32 23.98) (end 273.82 24.48) (width 1) (layer "B.Cu") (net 2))
 (segment (start 274.32 20.32) (end 274.32 23.98) (width 1) (layer "B.Cu") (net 2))
 (segment (start 261.62 20.32) (end 261.62 24.48) (width 1) (layer "B.Cu") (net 3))
 (segment (start 273.82 38.1) (end 273.82 36.48) (width 1) (layer "B.Cu") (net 5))
 (segment (start 274.32 38.6) (end 274.32 40.64) (width 1) (layer "B.Cu") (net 5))
 (segment (start 273.82 38.1) (end 274.32 38.6) (width 1) (layer "B.Cu") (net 5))
 (segment (start 273.117919 30.48) (end 275.82 30.48) (width 1) (layer "B.Cu") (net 1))
 (segment (start 264.16 20.32) (end 264.16 21.522081) (width 1) (layer "B.Cu") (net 1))
 (segment (start 264.16 21.522081) (end 273.117919 30.48) (width 1) (layer "B.Cu") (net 1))
 (segment (start 261.62 36.48) (end 261.62 40.64) (width 1) (layer "B.Cu") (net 4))
 (segment (start 246.58762 72.939991) (end 246.58762 74.639991) (width 0.6) (layer "B.Cu") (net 26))
 (segment (start 239.947611 81.28) (end 238.206498 81.28) (width 0.6) (layer "B.Cu") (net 26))
 (segment (start 246.58762 74.639991) (end 239.947611 81.28) (width 0.6) (layer "B.Cu") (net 26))
 (segment (start 239.18762 77.758878) (end 238.206498 78.74) (width 0.6) (layer "B.Cu") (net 25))
 (segment (start 239.18762 74.939991) (end 239.18762 77.758878) (width 0.6) (layer "B.Cu") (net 25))
 (segment (start 245.107611 83.82) (end 238.206498 83.82) (width 0.6) (layer "B.Cu") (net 27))
 (segment (start 246.58762 82.339991) (end 245.107611 83.82) (width 0.6) (layer "B.Cu") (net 27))
 (segment (start 186.255512 97.915614) (end 187.459898 99.12) (width 0.6) (layer "B.Cu") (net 31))
 (segment (start 187.459898 99.12) (end 198.835516 99.12) (width 0.6) (layer "B.Cu") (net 31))
 (segment (start 198.835516 99.12) (end 202.713249 95.242267) (width 0.6) (layer "B.Cu") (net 31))
 (segment (start 186.255512 93.21) (end 186.255512 97.915614) (width 0.6) (layer "B.Cu") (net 31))
 (segment (start 198.745982 107.505) (end 202.713249 111.472267) (width 0.6) (layer "B.Cu") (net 32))
 (segment (start 186.255512 113.415) (end 186.255512 108.792034) (width 0.6) (layer "B.Cu") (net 32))
 (segment (start 186.255512 108.792034) (end 187.542546 107.505) (width 0.6) (layer "B.Cu") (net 32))
 (segment (start 187.542546 107.505) (end 198.745982 107.505) (width 0.6) (layer "B.Cu") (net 32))
 (segment (start 196.363249 95.242267) (end 190.073245 95.242267) (width 0.6) (layer "B.Cu") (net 33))
 (segment (start 190.073245 95.242267) (end 188.795512 96.52) (width 0.6) (layer "B.Cu") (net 33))
 (segment (start 202.870982 105.28) (end 209.063249 111.472267) (width 0.6) (layer "B.Cu") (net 36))
 (segment (start 183.715512 110.105) (end 183.715512 108.005) (width 0.6) (layer "B.Cu") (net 36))
 (segment (start 183.715512 108.005) (end 186.440512 105.28) (width 0.6) (layer "B.Cu") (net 36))
 (segment (start 186.440512 105.28) (end 202.870982 105.28) (width 0.6) (layer "B.Cu") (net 36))
 (segment (start 183.715512 98.62) (end 183.715512 96.52) (width 0.6) (layer "B.Cu") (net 35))
 (segment (start 209.063249 95.242267) (end 203.69759 100.607926) (width 0.6) (layer "B.Cu") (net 35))
 (segment (start 185.703438 100.607926) (end 183.715512 98.62) (width 0.6) (layer "B.Cu") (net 35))
 (segment (start 203.69759 100.607926) (end 185.703438 100.607926) (width 0.6) (layer "B.Cu") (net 35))
 (segment (start 194.995982 110.105) (end 196.363249 111.472267) (width 0.6) (layer "B.Cu") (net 34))
 (segment (start 188.795512 110.105) (end 194.995982 110.105) (width 0.6) (layer "B.Cu") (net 34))
 (segment (start 256.383019 120.551981) (end 256.53 120.405) (width 1) (layer "B.Cu") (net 28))
 (segment (start 256.383019 125.263209) (end 256.383019 120.551981) (width 1) (layer "B.Cu") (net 28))
 (segment (start 251.303019 125.263209) (end 251.46 125.106228) (width 1) (layer "B.Cu") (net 29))
 (segment (start 251.46 123.7417) (end 250.23 122.5117) (width 1) (layer "B.Cu") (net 29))
 (segment (start 251.46 125.106228) (end 251.46 123.7417) (width 1) (layer "B.Cu") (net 29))
 (segment (start 250.23 122.5117) (end 250.23 120.405) (width 1) (layer "B.Cu") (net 29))
 (segment (start 253.843019 128.573209) (end 253.843019 115.818019) (width 1) (layer "B.Cu") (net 30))
 (segment (start 253.843019 115.818019) (end 253.63 115.605) (width 1) (layer "B.Cu") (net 30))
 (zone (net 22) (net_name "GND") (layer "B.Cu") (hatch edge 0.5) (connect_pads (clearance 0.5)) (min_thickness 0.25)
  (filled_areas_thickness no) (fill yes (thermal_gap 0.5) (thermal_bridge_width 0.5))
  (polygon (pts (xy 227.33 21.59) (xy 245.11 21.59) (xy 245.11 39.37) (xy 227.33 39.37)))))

